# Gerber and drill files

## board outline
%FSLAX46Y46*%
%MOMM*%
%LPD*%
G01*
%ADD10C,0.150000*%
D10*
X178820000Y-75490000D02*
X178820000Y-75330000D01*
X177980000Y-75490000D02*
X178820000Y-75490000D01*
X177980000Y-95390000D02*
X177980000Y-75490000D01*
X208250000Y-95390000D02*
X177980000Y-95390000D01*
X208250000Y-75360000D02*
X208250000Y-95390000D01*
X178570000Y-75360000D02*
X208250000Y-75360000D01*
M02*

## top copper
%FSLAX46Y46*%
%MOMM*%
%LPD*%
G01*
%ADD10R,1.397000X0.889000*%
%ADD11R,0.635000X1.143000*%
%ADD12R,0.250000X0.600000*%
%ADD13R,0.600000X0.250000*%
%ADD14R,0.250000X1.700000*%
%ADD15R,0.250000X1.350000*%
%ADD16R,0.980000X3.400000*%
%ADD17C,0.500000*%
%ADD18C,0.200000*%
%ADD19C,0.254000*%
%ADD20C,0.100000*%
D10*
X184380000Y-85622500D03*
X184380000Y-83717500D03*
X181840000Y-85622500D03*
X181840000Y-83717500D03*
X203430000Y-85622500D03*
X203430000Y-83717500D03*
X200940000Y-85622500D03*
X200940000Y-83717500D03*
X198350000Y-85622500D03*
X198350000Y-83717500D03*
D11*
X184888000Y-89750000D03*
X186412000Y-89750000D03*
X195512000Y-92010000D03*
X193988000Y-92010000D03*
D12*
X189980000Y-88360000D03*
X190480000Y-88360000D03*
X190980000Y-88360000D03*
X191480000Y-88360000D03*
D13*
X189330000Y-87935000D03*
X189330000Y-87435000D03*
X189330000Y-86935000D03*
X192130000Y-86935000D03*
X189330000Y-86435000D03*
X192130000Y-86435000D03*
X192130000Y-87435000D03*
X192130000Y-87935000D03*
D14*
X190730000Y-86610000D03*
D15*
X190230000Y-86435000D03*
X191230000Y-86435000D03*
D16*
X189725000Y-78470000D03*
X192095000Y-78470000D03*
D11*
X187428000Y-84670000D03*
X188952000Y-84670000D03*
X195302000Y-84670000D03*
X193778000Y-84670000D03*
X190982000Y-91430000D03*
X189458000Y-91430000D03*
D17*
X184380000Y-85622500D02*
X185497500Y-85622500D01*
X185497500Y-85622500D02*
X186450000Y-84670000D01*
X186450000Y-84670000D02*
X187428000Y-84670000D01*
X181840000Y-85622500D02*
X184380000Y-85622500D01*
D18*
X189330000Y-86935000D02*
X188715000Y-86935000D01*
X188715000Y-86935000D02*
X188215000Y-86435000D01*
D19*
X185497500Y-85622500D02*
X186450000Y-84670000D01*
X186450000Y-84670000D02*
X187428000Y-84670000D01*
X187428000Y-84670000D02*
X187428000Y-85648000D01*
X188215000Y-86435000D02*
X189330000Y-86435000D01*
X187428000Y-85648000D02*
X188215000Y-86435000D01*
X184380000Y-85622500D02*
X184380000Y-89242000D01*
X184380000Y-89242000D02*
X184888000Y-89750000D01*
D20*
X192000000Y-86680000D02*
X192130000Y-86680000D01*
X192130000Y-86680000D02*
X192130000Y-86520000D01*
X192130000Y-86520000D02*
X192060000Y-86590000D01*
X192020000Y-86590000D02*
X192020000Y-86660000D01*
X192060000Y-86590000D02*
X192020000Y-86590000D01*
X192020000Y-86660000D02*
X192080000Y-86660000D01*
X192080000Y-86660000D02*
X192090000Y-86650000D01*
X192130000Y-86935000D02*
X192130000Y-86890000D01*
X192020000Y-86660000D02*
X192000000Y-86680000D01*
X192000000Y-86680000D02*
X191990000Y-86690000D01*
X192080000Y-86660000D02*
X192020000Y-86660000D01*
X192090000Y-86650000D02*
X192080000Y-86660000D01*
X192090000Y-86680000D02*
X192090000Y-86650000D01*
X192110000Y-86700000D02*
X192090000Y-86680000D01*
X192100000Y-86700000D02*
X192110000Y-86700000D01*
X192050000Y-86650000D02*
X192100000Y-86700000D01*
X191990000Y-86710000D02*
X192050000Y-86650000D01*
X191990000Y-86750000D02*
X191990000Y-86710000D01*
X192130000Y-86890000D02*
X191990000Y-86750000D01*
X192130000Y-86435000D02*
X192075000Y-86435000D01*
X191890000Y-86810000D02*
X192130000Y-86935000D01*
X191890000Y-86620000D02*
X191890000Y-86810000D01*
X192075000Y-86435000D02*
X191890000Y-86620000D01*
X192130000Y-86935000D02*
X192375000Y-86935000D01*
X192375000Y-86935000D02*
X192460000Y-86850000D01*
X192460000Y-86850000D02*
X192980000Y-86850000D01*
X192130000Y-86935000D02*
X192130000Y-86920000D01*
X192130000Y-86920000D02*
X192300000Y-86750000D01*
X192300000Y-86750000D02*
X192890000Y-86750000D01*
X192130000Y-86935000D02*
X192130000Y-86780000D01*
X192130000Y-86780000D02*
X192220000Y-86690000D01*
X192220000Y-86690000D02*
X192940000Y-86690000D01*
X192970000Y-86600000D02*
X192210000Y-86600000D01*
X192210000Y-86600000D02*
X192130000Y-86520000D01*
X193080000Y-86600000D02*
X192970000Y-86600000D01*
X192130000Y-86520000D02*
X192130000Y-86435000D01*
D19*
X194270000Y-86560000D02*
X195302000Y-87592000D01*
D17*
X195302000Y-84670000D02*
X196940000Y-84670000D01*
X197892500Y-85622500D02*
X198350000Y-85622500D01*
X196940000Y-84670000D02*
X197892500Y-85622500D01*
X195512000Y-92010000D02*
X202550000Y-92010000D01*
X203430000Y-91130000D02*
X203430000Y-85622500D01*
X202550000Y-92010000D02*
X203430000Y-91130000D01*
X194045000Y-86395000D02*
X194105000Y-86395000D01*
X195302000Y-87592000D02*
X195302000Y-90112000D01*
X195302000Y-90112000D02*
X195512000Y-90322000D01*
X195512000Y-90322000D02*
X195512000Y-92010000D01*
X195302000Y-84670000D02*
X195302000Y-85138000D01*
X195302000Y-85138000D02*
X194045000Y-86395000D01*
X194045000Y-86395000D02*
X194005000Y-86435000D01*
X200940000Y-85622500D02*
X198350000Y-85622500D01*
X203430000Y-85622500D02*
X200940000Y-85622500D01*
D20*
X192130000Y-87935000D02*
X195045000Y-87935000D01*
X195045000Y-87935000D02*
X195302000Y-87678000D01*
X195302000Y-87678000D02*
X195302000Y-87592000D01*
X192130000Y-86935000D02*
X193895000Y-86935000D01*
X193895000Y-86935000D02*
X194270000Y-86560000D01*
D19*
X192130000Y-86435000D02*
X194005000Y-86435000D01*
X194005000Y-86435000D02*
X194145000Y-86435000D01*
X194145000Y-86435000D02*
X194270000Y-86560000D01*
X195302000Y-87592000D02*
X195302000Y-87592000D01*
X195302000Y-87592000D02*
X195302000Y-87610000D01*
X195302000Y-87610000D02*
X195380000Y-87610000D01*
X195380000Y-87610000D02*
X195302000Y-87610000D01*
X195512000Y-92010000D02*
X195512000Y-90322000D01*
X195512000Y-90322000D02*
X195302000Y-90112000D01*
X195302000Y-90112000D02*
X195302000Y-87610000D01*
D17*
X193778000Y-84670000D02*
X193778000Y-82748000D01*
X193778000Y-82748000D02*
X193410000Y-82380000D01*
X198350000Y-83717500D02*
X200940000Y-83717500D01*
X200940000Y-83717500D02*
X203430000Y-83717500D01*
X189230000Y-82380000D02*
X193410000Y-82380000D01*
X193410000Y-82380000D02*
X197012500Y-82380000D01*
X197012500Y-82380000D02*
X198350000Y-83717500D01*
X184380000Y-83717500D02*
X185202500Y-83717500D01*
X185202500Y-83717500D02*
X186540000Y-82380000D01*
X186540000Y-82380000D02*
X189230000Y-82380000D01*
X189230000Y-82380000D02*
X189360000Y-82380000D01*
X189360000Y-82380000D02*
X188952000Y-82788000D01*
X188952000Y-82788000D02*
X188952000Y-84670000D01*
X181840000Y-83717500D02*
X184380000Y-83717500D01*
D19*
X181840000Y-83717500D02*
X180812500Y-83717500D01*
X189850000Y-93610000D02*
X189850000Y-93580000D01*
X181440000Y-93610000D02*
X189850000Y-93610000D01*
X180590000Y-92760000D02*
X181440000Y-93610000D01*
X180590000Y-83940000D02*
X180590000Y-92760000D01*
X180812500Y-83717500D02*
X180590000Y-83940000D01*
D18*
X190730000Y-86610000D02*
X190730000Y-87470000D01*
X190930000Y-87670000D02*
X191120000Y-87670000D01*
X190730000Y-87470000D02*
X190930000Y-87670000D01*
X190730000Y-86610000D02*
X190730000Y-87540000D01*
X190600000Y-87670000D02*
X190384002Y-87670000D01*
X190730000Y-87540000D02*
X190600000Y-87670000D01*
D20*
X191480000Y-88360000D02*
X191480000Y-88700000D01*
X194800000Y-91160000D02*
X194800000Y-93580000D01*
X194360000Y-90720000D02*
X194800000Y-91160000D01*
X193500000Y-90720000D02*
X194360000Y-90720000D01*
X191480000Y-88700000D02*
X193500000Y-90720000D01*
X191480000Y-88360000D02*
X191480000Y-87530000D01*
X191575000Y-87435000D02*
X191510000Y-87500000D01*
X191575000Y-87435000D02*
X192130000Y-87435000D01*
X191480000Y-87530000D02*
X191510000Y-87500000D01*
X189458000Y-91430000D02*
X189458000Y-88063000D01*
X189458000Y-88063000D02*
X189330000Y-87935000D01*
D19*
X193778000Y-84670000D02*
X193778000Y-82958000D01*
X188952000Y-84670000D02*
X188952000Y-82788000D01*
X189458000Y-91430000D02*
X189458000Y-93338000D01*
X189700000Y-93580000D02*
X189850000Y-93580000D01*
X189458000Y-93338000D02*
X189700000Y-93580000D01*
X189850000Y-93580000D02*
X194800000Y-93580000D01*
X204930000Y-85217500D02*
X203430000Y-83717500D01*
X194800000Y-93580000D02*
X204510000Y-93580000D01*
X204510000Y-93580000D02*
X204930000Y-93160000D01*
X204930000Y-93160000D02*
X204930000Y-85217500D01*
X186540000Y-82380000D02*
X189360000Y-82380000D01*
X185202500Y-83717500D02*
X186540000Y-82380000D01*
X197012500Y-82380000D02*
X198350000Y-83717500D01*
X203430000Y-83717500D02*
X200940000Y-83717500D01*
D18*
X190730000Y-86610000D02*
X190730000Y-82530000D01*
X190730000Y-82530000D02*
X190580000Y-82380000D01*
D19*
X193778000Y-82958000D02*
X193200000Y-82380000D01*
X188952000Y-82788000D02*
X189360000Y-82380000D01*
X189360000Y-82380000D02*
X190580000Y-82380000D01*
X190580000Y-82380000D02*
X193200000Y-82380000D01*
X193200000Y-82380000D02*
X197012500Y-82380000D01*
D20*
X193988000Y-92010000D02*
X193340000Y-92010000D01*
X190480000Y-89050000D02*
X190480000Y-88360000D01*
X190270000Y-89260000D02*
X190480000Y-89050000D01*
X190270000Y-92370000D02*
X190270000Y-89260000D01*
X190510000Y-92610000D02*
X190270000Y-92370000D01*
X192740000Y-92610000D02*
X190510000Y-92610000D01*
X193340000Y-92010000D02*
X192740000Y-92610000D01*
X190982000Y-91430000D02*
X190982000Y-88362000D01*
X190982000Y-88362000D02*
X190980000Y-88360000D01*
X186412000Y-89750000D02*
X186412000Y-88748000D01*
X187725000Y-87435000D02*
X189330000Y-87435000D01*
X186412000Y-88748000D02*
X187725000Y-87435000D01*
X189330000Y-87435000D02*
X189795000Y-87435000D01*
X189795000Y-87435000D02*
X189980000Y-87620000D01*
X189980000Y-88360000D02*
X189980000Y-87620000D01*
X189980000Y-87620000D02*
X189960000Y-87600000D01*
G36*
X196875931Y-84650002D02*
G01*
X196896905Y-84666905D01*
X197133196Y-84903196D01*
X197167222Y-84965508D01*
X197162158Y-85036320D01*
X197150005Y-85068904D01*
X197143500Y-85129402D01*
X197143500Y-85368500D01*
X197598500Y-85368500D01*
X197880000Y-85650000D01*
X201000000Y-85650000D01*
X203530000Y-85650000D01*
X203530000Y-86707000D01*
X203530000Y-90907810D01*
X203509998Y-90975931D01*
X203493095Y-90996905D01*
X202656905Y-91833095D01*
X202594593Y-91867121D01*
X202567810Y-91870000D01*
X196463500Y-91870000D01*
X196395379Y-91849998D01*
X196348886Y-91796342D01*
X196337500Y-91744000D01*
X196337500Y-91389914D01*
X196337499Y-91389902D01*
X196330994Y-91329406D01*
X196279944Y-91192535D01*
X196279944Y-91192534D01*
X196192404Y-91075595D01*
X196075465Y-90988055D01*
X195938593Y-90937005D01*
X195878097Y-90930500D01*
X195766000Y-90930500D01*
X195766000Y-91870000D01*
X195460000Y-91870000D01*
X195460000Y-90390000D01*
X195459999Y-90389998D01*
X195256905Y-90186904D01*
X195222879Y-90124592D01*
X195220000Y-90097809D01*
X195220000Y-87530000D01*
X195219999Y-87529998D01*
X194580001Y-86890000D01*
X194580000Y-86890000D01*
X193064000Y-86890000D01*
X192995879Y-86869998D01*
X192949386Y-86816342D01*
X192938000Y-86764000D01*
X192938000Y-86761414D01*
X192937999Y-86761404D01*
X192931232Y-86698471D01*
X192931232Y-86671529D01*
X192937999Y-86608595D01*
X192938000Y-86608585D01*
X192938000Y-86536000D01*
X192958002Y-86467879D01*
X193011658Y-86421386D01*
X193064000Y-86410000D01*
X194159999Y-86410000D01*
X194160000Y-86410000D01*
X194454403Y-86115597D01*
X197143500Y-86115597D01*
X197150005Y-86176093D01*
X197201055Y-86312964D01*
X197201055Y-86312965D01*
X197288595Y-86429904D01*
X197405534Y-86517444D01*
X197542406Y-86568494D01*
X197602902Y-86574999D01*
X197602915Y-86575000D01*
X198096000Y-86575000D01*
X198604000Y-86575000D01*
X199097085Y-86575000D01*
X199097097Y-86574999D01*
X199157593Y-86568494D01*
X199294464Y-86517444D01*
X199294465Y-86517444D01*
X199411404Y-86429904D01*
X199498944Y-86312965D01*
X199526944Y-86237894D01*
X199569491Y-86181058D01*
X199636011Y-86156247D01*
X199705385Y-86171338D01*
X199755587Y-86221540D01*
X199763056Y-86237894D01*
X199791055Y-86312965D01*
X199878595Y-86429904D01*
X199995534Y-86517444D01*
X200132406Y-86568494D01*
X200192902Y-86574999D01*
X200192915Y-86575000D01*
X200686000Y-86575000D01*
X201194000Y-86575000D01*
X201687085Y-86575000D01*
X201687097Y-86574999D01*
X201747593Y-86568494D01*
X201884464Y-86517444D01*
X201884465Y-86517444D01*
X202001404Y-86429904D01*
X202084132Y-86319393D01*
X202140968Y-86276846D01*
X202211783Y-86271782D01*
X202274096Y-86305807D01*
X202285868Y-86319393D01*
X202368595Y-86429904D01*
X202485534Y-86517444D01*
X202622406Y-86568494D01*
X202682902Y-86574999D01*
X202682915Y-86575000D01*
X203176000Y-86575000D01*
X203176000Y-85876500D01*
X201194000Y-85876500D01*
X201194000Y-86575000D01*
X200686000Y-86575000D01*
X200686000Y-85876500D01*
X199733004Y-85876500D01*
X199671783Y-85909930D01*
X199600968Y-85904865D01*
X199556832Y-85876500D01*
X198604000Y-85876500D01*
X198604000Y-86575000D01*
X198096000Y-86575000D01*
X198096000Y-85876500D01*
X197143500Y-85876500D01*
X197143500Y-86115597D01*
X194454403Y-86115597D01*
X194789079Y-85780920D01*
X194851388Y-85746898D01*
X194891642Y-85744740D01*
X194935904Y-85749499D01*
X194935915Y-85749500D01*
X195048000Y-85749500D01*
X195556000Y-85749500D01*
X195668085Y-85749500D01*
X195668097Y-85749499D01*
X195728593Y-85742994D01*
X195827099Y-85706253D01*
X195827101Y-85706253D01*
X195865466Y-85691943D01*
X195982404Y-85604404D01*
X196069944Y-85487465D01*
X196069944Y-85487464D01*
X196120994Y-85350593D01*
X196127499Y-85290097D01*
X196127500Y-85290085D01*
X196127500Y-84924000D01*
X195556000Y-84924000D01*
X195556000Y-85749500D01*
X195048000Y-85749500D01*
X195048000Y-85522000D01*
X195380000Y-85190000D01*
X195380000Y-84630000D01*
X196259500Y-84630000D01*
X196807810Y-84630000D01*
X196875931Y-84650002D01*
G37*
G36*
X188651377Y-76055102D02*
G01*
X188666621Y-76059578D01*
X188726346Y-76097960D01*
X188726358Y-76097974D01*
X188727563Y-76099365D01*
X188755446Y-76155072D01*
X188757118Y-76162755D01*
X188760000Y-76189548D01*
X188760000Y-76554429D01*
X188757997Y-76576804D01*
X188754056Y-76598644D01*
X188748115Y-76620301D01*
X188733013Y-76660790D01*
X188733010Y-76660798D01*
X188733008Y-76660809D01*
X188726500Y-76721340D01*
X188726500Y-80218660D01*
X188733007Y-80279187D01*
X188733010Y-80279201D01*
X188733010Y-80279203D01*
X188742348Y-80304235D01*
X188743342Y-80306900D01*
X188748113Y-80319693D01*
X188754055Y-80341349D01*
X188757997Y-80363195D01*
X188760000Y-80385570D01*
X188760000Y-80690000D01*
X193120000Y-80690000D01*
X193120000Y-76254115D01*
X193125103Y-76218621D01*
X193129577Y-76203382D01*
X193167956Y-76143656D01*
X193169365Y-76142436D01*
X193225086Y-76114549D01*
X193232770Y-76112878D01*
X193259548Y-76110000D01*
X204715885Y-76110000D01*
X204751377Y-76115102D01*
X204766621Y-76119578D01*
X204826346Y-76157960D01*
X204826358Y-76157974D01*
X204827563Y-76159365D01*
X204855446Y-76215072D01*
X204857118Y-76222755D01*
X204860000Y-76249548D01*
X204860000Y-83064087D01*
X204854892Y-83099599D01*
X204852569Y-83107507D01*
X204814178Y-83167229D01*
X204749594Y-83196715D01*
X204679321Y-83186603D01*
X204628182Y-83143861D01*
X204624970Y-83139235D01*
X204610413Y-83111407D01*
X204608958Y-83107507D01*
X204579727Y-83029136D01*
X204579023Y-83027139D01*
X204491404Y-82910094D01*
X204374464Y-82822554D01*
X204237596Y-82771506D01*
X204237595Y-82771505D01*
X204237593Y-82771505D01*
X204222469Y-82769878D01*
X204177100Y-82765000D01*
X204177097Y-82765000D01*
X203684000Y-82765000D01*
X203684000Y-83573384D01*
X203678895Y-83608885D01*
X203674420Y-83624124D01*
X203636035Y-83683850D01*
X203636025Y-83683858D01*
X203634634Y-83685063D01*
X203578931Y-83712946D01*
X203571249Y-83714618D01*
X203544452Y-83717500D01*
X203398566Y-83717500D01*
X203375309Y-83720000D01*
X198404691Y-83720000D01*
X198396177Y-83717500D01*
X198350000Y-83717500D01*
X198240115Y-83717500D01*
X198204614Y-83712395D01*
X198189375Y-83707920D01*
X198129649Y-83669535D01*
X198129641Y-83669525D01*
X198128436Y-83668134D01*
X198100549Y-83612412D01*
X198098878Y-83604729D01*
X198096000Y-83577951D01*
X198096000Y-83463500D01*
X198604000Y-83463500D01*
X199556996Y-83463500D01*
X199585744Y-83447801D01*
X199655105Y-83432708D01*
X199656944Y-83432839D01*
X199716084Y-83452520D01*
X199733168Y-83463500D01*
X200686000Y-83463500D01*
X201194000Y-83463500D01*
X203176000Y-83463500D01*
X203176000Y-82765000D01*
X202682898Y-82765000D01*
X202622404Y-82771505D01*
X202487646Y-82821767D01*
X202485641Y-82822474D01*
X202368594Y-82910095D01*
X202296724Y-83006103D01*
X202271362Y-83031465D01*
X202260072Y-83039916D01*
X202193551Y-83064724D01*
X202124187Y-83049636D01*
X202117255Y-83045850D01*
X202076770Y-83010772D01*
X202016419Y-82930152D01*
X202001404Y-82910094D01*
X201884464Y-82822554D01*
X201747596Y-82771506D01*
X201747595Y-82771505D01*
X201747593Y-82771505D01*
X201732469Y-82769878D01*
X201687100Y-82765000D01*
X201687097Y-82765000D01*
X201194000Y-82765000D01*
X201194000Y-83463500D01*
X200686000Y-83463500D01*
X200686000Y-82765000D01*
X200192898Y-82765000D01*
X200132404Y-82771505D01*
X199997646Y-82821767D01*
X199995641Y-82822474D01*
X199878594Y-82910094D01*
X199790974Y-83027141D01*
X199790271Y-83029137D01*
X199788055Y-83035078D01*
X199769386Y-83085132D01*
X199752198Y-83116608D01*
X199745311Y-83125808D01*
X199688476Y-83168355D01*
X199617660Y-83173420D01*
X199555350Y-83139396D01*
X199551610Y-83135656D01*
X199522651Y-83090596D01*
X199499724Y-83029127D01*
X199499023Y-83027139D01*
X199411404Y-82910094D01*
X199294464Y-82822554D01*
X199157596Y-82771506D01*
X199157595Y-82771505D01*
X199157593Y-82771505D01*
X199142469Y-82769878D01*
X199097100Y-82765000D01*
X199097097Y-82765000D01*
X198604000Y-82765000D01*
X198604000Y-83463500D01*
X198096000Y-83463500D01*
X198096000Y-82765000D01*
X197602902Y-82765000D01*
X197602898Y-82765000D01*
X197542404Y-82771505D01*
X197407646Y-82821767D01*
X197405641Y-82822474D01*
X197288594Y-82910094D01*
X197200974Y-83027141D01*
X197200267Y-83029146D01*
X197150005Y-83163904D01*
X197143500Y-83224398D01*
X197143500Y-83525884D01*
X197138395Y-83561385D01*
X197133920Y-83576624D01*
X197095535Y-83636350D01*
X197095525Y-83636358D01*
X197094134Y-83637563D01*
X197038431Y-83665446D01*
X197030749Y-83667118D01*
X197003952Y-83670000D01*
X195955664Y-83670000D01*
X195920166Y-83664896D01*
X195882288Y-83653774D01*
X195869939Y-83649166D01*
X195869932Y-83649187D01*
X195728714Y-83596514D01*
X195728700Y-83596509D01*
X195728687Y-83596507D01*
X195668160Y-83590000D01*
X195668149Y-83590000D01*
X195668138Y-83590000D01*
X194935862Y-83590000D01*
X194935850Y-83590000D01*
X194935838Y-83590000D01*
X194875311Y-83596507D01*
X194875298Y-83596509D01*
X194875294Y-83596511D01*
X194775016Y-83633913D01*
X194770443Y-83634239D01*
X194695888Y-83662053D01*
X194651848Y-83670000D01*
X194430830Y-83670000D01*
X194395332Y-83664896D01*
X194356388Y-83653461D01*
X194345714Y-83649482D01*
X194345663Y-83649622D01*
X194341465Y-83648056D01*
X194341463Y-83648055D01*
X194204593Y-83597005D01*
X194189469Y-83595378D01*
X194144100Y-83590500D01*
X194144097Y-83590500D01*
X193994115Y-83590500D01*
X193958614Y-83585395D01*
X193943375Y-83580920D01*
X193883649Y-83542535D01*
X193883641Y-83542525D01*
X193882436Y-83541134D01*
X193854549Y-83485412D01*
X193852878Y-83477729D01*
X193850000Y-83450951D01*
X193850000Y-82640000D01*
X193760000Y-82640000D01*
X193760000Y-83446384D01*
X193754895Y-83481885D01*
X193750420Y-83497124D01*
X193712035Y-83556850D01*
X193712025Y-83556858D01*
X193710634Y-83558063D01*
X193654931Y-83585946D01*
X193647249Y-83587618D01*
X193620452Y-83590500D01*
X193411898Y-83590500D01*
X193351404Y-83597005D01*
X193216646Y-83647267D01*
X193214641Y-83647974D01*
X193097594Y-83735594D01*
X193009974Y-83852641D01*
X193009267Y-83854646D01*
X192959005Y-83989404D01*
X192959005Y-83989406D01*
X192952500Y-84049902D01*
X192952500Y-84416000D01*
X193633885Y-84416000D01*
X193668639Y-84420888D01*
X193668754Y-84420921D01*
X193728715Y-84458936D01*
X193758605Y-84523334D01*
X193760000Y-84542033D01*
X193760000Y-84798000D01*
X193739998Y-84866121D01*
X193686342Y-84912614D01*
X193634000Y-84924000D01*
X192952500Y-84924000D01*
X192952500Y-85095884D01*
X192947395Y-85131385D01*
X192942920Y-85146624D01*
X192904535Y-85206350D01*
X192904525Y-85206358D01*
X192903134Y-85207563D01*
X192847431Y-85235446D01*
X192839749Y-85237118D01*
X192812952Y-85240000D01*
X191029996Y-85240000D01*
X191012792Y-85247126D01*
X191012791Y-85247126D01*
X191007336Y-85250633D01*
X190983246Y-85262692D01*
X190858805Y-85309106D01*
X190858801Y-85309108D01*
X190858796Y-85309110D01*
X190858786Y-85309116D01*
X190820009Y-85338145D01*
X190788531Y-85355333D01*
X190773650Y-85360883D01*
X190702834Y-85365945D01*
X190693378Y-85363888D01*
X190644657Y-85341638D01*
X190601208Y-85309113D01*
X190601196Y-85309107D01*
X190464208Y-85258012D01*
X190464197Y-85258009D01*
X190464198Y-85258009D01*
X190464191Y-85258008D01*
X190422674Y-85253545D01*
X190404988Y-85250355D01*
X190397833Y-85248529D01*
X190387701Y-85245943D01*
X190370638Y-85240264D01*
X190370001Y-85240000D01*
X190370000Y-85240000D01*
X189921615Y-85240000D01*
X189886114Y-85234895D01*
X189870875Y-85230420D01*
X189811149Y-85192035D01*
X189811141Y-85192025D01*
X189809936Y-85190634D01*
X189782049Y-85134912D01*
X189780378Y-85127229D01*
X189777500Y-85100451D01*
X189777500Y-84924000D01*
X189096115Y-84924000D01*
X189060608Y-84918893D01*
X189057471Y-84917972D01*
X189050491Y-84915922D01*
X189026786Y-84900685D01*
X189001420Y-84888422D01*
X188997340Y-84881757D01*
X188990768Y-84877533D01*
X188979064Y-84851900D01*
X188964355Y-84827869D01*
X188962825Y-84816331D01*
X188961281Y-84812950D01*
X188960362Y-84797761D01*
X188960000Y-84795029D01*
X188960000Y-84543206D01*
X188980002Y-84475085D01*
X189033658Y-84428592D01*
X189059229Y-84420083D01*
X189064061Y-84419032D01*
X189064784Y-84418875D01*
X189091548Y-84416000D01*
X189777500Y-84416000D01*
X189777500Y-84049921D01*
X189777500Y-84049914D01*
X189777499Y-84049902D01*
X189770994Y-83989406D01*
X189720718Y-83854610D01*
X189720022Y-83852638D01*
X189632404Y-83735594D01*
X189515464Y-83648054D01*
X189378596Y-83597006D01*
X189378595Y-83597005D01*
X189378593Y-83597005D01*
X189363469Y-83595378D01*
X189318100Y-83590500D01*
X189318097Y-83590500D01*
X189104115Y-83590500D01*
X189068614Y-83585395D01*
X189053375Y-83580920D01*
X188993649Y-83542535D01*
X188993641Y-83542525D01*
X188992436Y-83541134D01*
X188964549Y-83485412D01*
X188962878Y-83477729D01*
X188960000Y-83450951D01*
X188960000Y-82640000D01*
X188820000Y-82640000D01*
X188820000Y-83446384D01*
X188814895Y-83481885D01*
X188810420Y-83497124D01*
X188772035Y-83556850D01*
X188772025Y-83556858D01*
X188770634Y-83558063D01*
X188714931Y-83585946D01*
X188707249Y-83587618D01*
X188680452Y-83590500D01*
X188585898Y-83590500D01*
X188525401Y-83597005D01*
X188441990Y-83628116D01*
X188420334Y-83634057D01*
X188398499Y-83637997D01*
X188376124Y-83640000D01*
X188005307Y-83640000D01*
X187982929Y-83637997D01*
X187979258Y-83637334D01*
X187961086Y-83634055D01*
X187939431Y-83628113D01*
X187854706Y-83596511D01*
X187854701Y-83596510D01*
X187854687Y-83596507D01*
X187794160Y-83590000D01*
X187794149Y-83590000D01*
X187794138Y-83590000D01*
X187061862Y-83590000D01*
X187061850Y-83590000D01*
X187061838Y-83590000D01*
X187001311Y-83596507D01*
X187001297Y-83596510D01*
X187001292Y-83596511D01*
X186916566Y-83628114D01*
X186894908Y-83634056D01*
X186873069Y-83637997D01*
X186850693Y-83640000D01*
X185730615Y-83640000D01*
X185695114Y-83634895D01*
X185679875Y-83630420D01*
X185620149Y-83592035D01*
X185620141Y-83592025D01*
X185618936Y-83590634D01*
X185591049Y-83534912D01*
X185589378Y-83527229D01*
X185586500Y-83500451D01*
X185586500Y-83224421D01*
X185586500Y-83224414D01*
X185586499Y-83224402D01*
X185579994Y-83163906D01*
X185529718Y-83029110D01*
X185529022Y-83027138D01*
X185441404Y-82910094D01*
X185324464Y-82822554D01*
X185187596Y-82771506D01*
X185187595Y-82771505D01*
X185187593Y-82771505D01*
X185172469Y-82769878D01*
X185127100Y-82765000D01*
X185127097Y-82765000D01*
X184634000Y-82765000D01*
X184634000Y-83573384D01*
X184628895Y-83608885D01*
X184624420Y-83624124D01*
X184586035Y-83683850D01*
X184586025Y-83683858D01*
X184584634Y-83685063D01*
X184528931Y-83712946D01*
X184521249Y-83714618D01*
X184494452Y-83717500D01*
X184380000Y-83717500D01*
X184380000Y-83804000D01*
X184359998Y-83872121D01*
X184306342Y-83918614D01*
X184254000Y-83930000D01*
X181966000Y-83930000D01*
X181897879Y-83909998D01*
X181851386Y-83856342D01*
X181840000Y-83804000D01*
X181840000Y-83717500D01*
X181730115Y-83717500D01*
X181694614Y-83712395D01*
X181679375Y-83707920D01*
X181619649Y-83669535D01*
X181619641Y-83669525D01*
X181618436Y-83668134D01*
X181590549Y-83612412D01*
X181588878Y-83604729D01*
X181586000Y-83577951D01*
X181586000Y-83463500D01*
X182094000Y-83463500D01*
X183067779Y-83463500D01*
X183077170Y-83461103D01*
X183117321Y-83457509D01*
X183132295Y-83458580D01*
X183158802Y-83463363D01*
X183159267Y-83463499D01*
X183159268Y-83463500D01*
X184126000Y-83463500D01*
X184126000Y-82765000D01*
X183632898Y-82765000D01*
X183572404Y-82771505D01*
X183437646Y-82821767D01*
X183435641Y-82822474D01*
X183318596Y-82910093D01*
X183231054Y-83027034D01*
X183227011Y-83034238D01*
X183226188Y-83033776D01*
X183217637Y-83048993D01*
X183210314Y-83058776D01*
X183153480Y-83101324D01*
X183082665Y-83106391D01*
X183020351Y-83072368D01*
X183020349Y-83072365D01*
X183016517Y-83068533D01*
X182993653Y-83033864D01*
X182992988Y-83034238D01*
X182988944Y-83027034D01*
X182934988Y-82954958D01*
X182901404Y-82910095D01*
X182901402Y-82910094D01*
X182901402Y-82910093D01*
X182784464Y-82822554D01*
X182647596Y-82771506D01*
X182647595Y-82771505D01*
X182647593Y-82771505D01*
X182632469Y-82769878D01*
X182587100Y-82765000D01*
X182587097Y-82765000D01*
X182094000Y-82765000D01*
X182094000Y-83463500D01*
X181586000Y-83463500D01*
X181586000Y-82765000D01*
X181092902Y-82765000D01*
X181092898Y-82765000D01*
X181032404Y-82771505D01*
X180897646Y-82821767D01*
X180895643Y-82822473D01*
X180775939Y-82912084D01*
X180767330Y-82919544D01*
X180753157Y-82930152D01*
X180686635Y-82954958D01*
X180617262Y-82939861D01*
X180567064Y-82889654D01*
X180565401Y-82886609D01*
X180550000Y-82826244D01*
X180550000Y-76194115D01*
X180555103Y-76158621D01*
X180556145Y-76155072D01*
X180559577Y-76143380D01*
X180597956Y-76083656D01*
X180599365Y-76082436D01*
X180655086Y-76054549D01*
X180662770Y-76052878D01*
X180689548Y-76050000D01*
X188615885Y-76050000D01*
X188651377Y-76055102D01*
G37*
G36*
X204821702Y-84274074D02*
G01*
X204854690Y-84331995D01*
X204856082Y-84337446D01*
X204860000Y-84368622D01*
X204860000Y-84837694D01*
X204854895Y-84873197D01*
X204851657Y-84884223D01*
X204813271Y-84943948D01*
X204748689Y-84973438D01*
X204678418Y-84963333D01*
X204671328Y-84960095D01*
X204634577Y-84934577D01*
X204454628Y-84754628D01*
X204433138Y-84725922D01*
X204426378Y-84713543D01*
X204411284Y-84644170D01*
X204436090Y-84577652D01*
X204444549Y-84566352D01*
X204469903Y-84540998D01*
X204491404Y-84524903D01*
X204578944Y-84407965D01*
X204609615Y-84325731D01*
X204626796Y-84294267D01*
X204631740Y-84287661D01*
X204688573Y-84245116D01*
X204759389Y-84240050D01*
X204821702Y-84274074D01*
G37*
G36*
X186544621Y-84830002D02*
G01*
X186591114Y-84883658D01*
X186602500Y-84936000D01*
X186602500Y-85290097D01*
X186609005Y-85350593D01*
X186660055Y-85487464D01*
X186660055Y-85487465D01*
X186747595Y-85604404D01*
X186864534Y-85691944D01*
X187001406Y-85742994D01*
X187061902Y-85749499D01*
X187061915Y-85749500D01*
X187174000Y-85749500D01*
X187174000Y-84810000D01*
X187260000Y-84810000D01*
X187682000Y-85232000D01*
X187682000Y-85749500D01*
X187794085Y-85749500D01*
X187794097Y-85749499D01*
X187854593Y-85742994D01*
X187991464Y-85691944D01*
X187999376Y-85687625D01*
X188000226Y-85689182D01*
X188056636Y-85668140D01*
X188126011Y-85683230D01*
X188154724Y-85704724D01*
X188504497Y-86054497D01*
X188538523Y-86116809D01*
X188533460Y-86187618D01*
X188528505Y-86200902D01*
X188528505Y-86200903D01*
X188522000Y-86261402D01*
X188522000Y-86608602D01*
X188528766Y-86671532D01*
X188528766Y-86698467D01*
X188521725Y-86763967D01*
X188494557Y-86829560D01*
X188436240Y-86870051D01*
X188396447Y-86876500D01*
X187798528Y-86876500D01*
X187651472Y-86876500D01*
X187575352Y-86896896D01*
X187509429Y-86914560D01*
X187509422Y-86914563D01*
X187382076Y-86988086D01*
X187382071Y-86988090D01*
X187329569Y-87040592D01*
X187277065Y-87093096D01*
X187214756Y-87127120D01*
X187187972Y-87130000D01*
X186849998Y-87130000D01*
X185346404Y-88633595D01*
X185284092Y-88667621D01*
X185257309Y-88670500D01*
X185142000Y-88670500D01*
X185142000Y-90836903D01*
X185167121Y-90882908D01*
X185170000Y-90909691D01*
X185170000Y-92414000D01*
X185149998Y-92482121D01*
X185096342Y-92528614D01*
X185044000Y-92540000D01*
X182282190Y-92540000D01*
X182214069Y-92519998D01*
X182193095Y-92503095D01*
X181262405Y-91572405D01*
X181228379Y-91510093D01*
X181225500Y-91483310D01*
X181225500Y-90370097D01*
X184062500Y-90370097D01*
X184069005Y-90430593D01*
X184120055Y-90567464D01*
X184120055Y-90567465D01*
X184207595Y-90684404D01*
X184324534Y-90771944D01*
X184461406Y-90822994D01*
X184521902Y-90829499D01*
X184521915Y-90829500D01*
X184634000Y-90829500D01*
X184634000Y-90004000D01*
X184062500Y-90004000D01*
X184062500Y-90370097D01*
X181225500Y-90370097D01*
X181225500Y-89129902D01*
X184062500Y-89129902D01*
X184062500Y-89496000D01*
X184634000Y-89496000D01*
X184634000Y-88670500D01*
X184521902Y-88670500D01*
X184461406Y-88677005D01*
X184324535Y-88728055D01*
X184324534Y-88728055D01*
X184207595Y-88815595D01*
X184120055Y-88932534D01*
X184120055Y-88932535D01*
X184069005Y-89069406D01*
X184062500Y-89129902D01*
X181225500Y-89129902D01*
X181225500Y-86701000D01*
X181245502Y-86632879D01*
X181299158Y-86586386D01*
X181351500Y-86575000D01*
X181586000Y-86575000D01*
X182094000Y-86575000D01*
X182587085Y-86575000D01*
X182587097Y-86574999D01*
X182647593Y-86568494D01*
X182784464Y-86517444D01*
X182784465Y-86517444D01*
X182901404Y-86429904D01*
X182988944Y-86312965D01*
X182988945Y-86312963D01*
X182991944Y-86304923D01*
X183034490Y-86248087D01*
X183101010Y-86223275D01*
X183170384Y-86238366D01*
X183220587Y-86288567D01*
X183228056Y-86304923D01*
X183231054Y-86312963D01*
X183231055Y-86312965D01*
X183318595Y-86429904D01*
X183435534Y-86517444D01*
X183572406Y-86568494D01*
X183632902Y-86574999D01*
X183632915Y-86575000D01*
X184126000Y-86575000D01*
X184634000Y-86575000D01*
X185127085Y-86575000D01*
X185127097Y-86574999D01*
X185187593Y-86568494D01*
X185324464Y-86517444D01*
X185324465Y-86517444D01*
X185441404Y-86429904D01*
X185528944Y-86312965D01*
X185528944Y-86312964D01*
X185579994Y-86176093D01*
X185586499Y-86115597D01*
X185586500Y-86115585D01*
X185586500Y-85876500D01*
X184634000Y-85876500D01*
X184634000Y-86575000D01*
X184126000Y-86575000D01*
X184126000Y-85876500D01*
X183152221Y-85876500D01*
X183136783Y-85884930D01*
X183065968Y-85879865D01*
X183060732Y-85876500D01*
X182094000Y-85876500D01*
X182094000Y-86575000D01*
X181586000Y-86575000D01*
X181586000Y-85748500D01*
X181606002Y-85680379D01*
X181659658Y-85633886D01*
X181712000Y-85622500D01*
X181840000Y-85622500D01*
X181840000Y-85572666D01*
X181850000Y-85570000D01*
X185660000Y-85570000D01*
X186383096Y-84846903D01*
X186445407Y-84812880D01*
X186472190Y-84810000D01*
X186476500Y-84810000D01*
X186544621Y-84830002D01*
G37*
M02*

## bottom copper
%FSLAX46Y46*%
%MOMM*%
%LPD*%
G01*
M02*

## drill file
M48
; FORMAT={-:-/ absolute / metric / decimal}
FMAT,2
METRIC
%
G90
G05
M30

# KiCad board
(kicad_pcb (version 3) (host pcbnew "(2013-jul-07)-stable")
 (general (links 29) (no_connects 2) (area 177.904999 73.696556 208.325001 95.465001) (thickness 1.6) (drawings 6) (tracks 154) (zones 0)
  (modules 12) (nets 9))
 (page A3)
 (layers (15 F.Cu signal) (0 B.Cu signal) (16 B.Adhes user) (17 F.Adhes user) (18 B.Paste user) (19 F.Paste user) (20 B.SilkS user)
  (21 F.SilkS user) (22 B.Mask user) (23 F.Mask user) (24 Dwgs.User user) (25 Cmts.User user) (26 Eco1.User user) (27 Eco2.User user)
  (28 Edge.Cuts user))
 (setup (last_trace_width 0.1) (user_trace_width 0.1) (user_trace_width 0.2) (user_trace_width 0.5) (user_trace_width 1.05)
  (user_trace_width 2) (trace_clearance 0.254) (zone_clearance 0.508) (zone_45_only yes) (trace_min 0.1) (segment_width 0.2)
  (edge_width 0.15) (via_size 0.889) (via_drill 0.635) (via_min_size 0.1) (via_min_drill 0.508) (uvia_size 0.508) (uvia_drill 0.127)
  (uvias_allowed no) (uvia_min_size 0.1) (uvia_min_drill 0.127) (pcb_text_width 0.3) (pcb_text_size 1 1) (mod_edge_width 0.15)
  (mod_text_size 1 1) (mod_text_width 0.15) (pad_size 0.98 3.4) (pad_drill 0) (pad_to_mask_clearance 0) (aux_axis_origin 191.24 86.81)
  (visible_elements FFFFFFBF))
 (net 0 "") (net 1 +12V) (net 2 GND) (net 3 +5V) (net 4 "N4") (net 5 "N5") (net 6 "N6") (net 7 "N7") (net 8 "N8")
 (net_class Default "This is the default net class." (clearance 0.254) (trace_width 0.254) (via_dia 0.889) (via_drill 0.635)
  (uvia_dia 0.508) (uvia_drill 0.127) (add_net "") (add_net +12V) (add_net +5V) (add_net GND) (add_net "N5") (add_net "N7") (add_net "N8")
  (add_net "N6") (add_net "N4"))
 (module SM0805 (layer F.Cu) (at 184.38 84.67 90)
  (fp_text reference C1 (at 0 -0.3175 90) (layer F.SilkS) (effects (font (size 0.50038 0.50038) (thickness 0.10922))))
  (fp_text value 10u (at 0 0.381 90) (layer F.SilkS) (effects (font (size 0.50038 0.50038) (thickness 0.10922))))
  (pad 1 smd rect (at -0.9525 0 90) (size 0.889 1.397) (layers F.Cu F.Paste F.Mask) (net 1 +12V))
  (pad 2 smd rect (at 0.9525 0 90) (size 0.889 1.397) (layers F.Cu F.Paste F.Mask) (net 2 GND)))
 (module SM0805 (layer F.Cu) (at 181.84 84.67 90)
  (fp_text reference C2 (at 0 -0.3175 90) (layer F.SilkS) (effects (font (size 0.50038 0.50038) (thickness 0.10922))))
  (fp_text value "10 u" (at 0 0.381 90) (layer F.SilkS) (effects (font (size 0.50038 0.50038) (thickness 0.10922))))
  (pad 1 smd rect (at -0.9525 0 90) (size 0.889 1.397) (layers F.Cu F.Paste F.Mask) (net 1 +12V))
  (pad 2 smd rect (at 0.9525 0 90) (size 0.889 1.397) (layers F.Cu F.Paste F.Mask) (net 2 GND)))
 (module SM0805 (layer F.Cu) (at 203.43 84.67 90)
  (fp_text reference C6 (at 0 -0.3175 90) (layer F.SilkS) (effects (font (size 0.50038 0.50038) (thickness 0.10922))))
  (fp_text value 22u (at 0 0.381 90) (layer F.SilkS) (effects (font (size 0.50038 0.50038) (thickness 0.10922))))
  (pad 1 smd rect (at -0.9525 0 90) (size 0.889 1.397) (layers F.Cu F.Paste F.Mask) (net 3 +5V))
  (pad 2 smd rect (at 0.9525 0 90) (size 0.889 1.397) (layers F.Cu F.Paste F.Mask) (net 2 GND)))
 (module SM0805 (layer F.Cu) (at 200.94 84.67 90)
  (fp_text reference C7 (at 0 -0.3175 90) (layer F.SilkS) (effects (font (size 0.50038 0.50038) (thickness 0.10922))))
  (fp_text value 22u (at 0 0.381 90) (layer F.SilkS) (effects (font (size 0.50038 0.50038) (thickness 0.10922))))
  (pad 1 smd rect (at -0.9525 0 90) (size 0.889 1.397) (layers F.Cu F.Paste F.Mask) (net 3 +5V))
  (pad 2 smd rect (at 0.9525 0 90) (size 0.889 1.397) (layers F.Cu F.Paste F.Mask) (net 2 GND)))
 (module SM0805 (layer F.Cu) (at 198.35 84.67 90)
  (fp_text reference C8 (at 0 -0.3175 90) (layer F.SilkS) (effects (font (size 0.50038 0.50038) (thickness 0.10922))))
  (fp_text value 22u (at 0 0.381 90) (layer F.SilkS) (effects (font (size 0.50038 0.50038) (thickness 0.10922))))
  (pad 1 smd rect (at -0.9525 0 90) (size 0.889 1.397) (layers F.Cu F.Paste F.Mask) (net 3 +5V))
  (pad 2 smd rect (at 0.9525 0 90) (size 0.889 1.397) (layers F.Cu F.Paste F.Mask) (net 2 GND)))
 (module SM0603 (layer F.Cu) (at 185.65 89.75)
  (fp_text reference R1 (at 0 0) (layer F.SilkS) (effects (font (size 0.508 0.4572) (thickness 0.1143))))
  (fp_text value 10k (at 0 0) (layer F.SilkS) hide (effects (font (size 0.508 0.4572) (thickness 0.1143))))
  (pad 1 smd rect (at -0.762 0) (size 0.635 1.143) (layers F.Cu F.Paste F.Mask) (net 1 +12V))
  (pad 2 smd rect (at 0.762 0) (size 0.635 1.143) (layers F.Cu F.Paste F.Mask) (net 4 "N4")))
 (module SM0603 (layer F.Cu) (at 194.75 92.01 180)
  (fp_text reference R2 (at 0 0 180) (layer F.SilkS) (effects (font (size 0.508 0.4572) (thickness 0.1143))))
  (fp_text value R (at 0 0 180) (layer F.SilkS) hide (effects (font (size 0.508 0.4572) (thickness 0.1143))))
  (pad 1 smd rect (at -0.762 0 180) (size 0.635 1.143) (layers F.Cu F.Paste F.Mask) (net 3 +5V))
  (pad 2 smd rect (at 0.762 0 180) (size 0.635 1.143) (layers F.Cu F.Paste F.Mask) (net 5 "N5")))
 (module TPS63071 (layer F.Cu) (at 190.73 87.21 90)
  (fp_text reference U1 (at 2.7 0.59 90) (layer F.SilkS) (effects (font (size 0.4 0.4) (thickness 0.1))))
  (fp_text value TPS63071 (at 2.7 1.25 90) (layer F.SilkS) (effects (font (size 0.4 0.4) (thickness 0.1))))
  (pad 1 smd rect (at -1.15 -0.75 90) (size 0.6 0.25) (layers F.Cu F.Paste F.Mask) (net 4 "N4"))
  (pad 2 smd rect (at -1.15 -0.25 90) (size 0.6 0.25) (layers F.Cu F.Paste F.Mask) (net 5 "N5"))
  (pad 3 smd rect (at -1.15 0.25 90) (size 0.6 0.25) (layers F.Cu F.Paste F.Mask) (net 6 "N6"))
  (pad 4 smd rect (at -1.15 0.75 90) (size 0.6 0.25) (layers F.Cu F.Paste F.Mask) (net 2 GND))
  (pad 15 smd rect (at -0.725 -1.4 90) (size 0.25 0.6) (layers F.Cu F.Paste F.Mask) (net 2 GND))
  (pad 14 smd rect (at -0.225 -1.4 90) (size 0.25 0.6) (layers F.Cu F.Paste F.Mask) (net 4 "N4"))
  (pad 13 smd rect (at 0.275 -1.4 90) (size 0.25 0.6) (layers F.Cu F.Paste F.Mask) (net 1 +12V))
  (pad 7 smd rect (at 0.275 1.4 90) (size 0.25 0.6) (layers F.Cu F.Paste F.Mask) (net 3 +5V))
  (pad 12 smd rect (at 0.775 -1.4 90) (size 0.25 0.6) (layers F.Cu F.Paste F.Mask) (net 1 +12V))
  (pad 8 smd rect (at 0.775 1.4 90) (size 0.25 0.6) (layers F.Cu F.Paste F.Mask) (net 3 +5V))
  (pad 6 smd rect (at -0.225 1.4 90) (size 0.25 0.6) (layers F.Cu F.Paste F.Mask) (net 2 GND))
  (pad 5 smd rect (at -0.725 1.4 90) (size 0.25 0.6) (layers F.Cu F.Paste F.Mask) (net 3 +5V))
  (pad 10 smd rect (at 0.6 0 90) (size 1.7 0.25) (layers F.Cu F.Paste F.Mask) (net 2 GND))
  (pad 11 smd rect (at 0.775 -0.5 90) (size 1.35 0.25) (layers F.Cu F.Paste F.Mask) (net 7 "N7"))
  (pad 9 smd rect (at 0.775 0.5 90) (size 1.35 0.25) (layers F.Cu F.Paste F.Mask) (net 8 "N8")))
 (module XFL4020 (layer F.Cu) (at 190.91 78.47)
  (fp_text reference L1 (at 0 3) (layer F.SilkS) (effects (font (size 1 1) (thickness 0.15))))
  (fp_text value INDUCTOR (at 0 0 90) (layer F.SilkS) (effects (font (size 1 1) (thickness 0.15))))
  (pad 1 smd rect (at -1.185 0) (size 0.98 3.4) (layers F.Cu F.Paste F.Mask) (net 7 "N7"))
  (pad 2 smd rect (at 1.185 0) (size 0.98 3.4) (layers F.Cu F.Paste F.Mask) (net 8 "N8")))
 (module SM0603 (layer F.Cu) (at 188.19 84.67)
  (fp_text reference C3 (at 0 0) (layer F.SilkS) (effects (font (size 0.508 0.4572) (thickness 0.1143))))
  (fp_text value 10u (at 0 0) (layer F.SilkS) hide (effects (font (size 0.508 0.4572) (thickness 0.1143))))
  (pad 1 smd rect (at -0.762 0) (size 0.635 1.143) (layers F.Cu F.Paste F.Mask) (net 1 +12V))
  (pad 2 smd rect (at 0.762 0) (size 0.635 1.143) (layers F.Cu F.Paste F.Mask) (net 2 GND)))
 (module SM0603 (layer F.Cu) (at 194.54 84.67 180)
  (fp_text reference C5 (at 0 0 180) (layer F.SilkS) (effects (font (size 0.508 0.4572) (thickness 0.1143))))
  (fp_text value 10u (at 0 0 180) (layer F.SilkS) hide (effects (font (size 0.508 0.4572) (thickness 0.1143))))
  (pad 1 smd rect (at -0.762 0 180) (size 0.635 1.143) (layers F.Cu F.Paste F.Mask) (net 3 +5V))
  (pad 2 smd rect (at 0.762 0 180) (size 0.635 1.143) (layers F.Cu F.Paste F.Mask) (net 2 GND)))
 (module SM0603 (layer F.Cu) (at 190.22 91.43 180)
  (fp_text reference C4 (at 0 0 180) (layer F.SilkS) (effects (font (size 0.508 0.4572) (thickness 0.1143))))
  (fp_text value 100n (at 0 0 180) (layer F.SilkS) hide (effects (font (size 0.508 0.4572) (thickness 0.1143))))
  (pad 1 smd rect (at -0.762 0 180) (size 0.635 1.143) (layers F.Cu F.Paste F.Mask) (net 6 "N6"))
  (pad 2 smd rect (at 0.762 0 180) (size 0.635 1.143) (layers F.Cu F.Paste F.Mask) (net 2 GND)))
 (gr_line (start 178.82 75.49) (end 178.82 75.33) (angle 90) (layer Edge.Cuts) (width 0.15))
 (gr_line (start 177.98 75.49) (end 178.82 75.49) (angle 90) (layer Edge.Cuts) (width 0.15))
 (gr_line (start 177.98 95.39) (end 177.98 75.49) (angle 90) (layer Edge.Cuts) (width 0.15))
 (gr_line (start 208.25 95.39) (end 177.98 95.39) (angle 90) (layer Edge.Cuts) (width 0.15))
 (gr_line (start 208.25 75.36) (end 208.25 95.39) (angle 90) (layer Edge.Cuts) (width 0.15))
 (gr_line (start 178.57 75.36) (end 208.25 75.36) (angle 90) (layer Edge.Cuts) (width 0.15))
 (segment (start 184.38 85.6225) (end 185.4975 85.6225) (width 0.5) (layer F.Cu) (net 1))
 (segment (start 185.4975 85.6225) (end 186.45 84.67) (width 0.5) (layer F.Cu) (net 1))
 (segment (start 186.45 84.67) (end 187.428 84.67) (width 0.5) (layer F.Cu) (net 1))
 (segment (start 181.84 85.6225) (end 184.38 85.6225) (width 0.5) (layer F.Cu) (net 1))
 (segment (start 189.33 86.935) (end 188.715 86.935) (width 0.2) (layer F.Cu) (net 1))
 (segment (start 188.715 86.935) (end 188.215 86.435) (width 0.2) (layer F.Cu) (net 1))
 (segment (start 185.4975 85.6225) (end 186.45 84.67) (width 0.254) (layer F.Cu) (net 1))
 (segment (start 186.45 84.67) (end 187.428 84.67) (width 0.254) (layer F.Cu) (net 1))
 (segment (start 187.428 84.67) (end 187.428 85.648) (width 0.254) (layer F.Cu) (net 1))
 (segment (start 188.215 86.435) (end 189.33 86.435) (width 0.254) (layer F.Cu) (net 1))
 (segment (start 187.428 85.648) (end 188.215 86.435) (width 0.254) (layer F.Cu) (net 1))
 (segment (start 184.38 85.6225) (end 184.38 89.242) (width 0.254) (layer F.Cu) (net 1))
 (segment (start 184.38 89.242) (end 184.888 89.75) (width 0.254) (layer F.Cu) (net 1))
 (segment (start 192 86.68) (end 192.13 86.68) (width 0.1) (layer F.Cu) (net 3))
 (segment (start 192.13 86.68) (end 192.13 86.52) (width 0.1) (layer F.Cu) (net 3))
 (segment (start 192.13 86.52) (end 192.06 86.59) (width 0.1) (layer F.Cu) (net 3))
 (segment (start 192.02 86.59) (end 192.02 86.66) (width 0.1) (layer F.Cu) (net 3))
 (segment (start 192.06 86.59) (end 192.02 86.59) (width 0.1) (layer F.Cu) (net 3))
 (segment (start 192.02 86.66) (end 192.08 86.66) (width 0.1) (layer F.Cu) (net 3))
 (segment (start 192.08 86.66) (end 192.09 86.65) (width 0.1) (layer F.Cu) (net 3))
 (segment (start 192.13 86.935) (end 192.13 86.89) (width 0.1) (layer F.Cu) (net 3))
 (segment (start 192.02 86.66) (end 192 86.68) (width 0.1) (layer F.Cu) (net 3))
 (segment (start 192 86.68) (end 191.99 86.69) (width 0.1) (layer F.Cu) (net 3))
 (segment (start 192.08 86.66) (end 192.02 86.66) (width 0.1) (layer F.Cu) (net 3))
 (segment (start 192.09 86.65) (end 192.08 86.66) (width 0.1) (layer F.Cu) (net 3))
 (segment (start 192.09 86.68) (end 192.09 86.65) (width 0.1) (layer F.Cu) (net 3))
 (segment (start 192.11 86.7) (end 192.09 86.68) (width 0.1) (layer F.Cu) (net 3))
 (segment (start 192.1 86.7) (end 192.11 86.7) (width 0.1) (layer F.Cu) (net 3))
 (segment (start 192.05 86.65) (end 192.1 86.7) (width 0.1) (layer F.Cu) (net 3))
 (segment (start 191.99 86.71) (end 192.05 86.65) (width 0.1) (layer F.Cu) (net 3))
 (segment (start 191.99 86.75) (end 191.99 86.71) (width 0.1) (layer F.Cu) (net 3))
 (segment (start 192.13 86.89) (end 191.99 86.75) (width 0.1) (layer F.Cu) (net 3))
 (segment (start 192.13 86.435) (end 192.075 86.435) (width 0.1) (layer F.Cu) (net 3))
 (segment (start 191.89 86.81) (end 192.13 86.935) (width 0.1) (layer F.Cu) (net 3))
 (segment (start 191.89 86.62) (end 191.89 86.81) (width 0.1) (layer F.Cu) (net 3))
 (segment (start 192.075 86.435) (end 191.89 86.62) (width 0.1) (layer F.Cu) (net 3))
 (segment (start 192.13 86.935) (end 192.375 86.935) (width 0.1) (layer F.Cu) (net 3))
 (segment (start 192.375 86.935) (end 192.46 86.85) (width 0.1) (layer F.Cu) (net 3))
 (segment (start 192.46 86.85) (end 192.98 86.85) (width 0.1) (layer F.Cu) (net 3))
 (segment (start 192.13 86.935) (end 192.13 86.92) (width 0.1) (layer F.Cu) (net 3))
 (segment (start 192.13 86.92) (end 192.3 86.75) (width 0.1) (layer F.Cu) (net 3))
 (segment (start 192.3 86.75) (end 192.89 86.75) (width 0.1) (layer F.Cu) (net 3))
 (segment (start 192.13 86.935) (end 192.13 86.78) (width 0.1) (layer F.Cu) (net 3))
 (segment (start 192.13 86.78) (end 192.22 86.69) (width 0.1) (layer F.Cu) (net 3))
 (segment (start 192.22 86.69) (end 192.94 86.69) (width 0.1) (layer F.Cu) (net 3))
 (segment (start 192.97 86.6) (end 192.21 86.6) (width 0.1) (layer F.Cu) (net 3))
 (segment (start 192.21 86.6) (end 192.13 86.52) (width 0.1) (layer F.Cu) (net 3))
 (segment (start 193.08 86.6) (end 192.97 86.6) (width 0.1) (layer F.Cu) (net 3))
 (segment (start 192.13 86.52) (end 192.13 86.435) (width 0.1) (layer F.Cu) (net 3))
 (segment (start 194.27 86.56) (end 195.302 87.592) (width 0.254) (layer F.Cu) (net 3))
 (segment (start 195.302 84.67) (end 196.94 84.67) (width 0.5) (layer F.Cu) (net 3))
 (segment (start 197.8925 85.6225) (end 198.35 85.6225) (width 0.5) (layer F.Cu) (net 3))
 (segment (start 196.94 84.67) (end 197.8925 85.6225) (width 0.5) (layer F.Cu) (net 3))
 (segment (start 195.512 92.01) (end 202.55 92.01) (width 0.5) (layer F.Cu) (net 3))
 (segment (start 203.43 91.13) (end 203.43 85.6225) (width 0.5) (layer F.Cu) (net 3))
 (segment (start 202.55 92.01) (end 203.43 91.13) (width 0.5) (layer F.Cu) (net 3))
 (segment (start 194.045 86.395) (end 194.105 86.395) (width 0.5) (layer F.Cu) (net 3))
 (segment (start 195.302 87.592) (end 195.302 90.112) (width 0.5) (layer F.Cu) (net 3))
 (segment (start 195.302 90.112) (end 195.512 90.322) (width 0.5) (layer F.Cu) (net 3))
 (segment (start 195.512 90.322) (end 195.512 92.01) (width 0.5) (layer F.Cu) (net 3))
 (segment (start 195.302 84.67) (end 195.302 85.138) (width 0.5) (layer F.Cu) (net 3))
 (segment (start 195.302 85.138) (end 194.045 86.395) (width 0.5) (layer F.Cu) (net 3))
 (segment (start 194.045 86.395) (end 194.005 86.435) (width 0.5) (layer F.Cu) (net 3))
 (segment (start 200.94 85.6225) (end 198.35 85.6225) (width 0.5) (layer F.Cu) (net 3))
 (segment (start 203.43 85.6225) (end 200.94 85.6225) (width 0.5) (layer F.Cu) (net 3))
 (segment (start 192.13 87.935) (end 195.045 87.935) (width 0.1) (layer F.Cu) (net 3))
 (segment (start 195.045 87.935) (end 195.302 87.678) (width 0.1) (layer F.Cu) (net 3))
 (segment (start 195.302 87.678) (end 195.302 87.592) (width 0.1) (layer F.Cu) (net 3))
 (segment (start 192.13 86.935) (end 193.895 86.935) (width 0.1) (layer F.Cu) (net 3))
 (segment (start 193.895 86.935) (end 194.27 86.56) (width 0.1) (layer F.Cu) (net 3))
 (segment (start 192.13 86.435) (end 194.005 86.435) (width 0.254) (layer F.Cu) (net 3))
 (segment (start 194.005 86.435) (end 194.145 86.435) (width 0.254) (layer F.Cu) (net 3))
 (segment (start 194.145 86.435) (end 194.27 86.56) (width 0.254) (layer F.Cu) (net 3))
 (segment (start 195.302 87.592) (end 195.302 87.592) (width 0.254) (layer F.Cu) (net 3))
 (segment (start 195.302 87.592) (end 195.302 87.61) (width 0.254) (layer F.Cu) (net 3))
 (segment (start 195.302 87.61) (end 195.38 87.61) (width 0.254) (layer F.Cu) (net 3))
 (segment (start 195.38 87.61) (end 195.302 87.61) (width 0.254) (layer F.Cu) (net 3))
 (segment (start 195.512 92.01) (end 195.512 90.322) (width 0.254) (layer F.Cu) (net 3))
 (segment (start 195.512 90.322) (end 195.302 90.112) (width 0.254) (layer F.Cu) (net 3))
 (segment (start 195.302 90.112) (end 195.302 87.61) (width 0.254) (layer F.Cu) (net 3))
 (segment (start 193.778 84.67) (end 193.778 82.748) (width 0.5) (layer F.Cu) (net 2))
 (segment (start 193.778 82.748) (end 193.41 82.38) (width 0.5) (layer F.Cu) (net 2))
 (segment (start 198.35 83.7175) (end 200.94 83.7175) (width 0.5) (layer F.Cu) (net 2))
 (segment (start 200.94 83.7175) (end 203.43 83.7175) (width 0.5) (layer F.Cu) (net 2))
 (segment (start 189.23 82.38) (end 193.41 82.38) (width 0.5) (layer F.Cu) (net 2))
 (segment (start 193.41 82.38) (end 197.0125 82.38) (width 0.5) (layer F.Cu) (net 2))
 (segment (start 197.0125 82.38) (end 198.35 83.7175) (width 0.5) (layer F.Cu) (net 2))
 (segment (start 184.38 83.7175) (end 185.2025 83.7175) (width 0.5) (layer F.Cu) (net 2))
 (segment (start 185.2025 83.7175) (end 186.54 82.38) (width 0.5) (layer F.Cu) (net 2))
 (segment (start 186.54 82.38) (end 189.23 82.38) (width 0.5) (layer F.Cu) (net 2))
 (segment (start 189.23 82.38) (end 189.36 82.38) (width 0.5) (layer F.Cu) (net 2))
 (segment (start 189.36 82.38) (end 188.952 82.788) (width 0.5) (layer F.Cu) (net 2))
 (segment (start 188.952 82.788) (end 188.952 84.67) (width 0.5) (layer F.Cu) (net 2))
 (segment (start 181.84 83.7175) (end 184.38 83.7175) (width 0.5) (layer F.Cu) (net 2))
 (segment (start 181.84 83.7175) (end 180.8125 83.7175) (width 0.254) (layer F.Cu) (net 2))
 (segment (start 189.85 93.61) (end 189.85 93.58) (width 0.254) (layer F.Cu) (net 2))
 (segment (start 181.44 93.61) (end 189.85 93.61) (width 0.254) (layer F.Cu) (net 2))
 (segment (start 180.59 92.76) (end 181.44 93.61) (width 0.254) (layer F.Cu) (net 2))
 (segment (start 180.59 83.94) (end 180.59 92.76) (width 0.254) (layer F.Cu) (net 2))
 (segment (start 180.8125 83.7175) (end 180.59 83.94) (width 0.254) (layer F.Cu) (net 2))
 (segment (start 190.73 86.61) (end 190.73 87.47) (width 0.2) (layer F.Cu) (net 2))
 (segment (start 190.93 87.67) (end 191.12 87.67) (width 0.2) (layer F.Cu) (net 2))
 (segment (start 190.73 87.47) (end 190.93 87.67) (width 0.2) (layer F.Cu) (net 2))
 (segment (start 190.73 86.61) (end 190.73 87.54) (width 0.2) (layer F.Cu) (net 2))
 (segment (start 190.6 87.67) (end 190.384002 87.67) (width 0.2) (layer F.Cu) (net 2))
 (segment (start 190.73 87.54) (end 190.6 87.67) (width 0.2) (layer F.Cu) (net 2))
 (segment (start 191.48 88.36) (end 191.48 88.7) (width 0.1) (layer F.Cu) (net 2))
 (segment (start 194.8 91.16) (end 194.8 93.58) (width 0.1) (layer F.Cu) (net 2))
 (segment (start 194.36 90.72) (end 194.8 91.16) (width 0.1) (layer F.Cu) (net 2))
 (segment (start 193.5 90.72) (end 194.36 90.72) (width 0.1) (layer F.Cu) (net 2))
 (segment (start 191.48 88.7) (end 193.5 90.72) (width 0.1) (layer F.Cu) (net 2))
 (segment (start 191.48 88.36) (end 191.48 87.53) (width 0.1) (layer F.Cu) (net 2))
 (segment (start 191.575 87.435) (end 191.51 87.5) (width 0.1) (layer F.Cu) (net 2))
 (segment (start 191.575 87.435) (end 192.13 87.435) (width 0.1) (layer F.Cu) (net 2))
 (segment (start 191.48 87.53) (end 191.51 87.5) (width 0.1) (layer F.Cu) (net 2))
 (segment (start 189.458 91.43) (end 189.458 88.063) (width 0.1) (layer F.Cu) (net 2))
 (segment (start 189.458 88.063) (end 189.33 87.935) (width 0.1) (layer F.Cu) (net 2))
 (segment (start 193.778 84.67) (end 193.778 82.958) (width 0.254) (layer F.Cu) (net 2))
 (segment (start 188.952 84.67) (end 188.952 82.788) (width 0.254) (layer F.Cu) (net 2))
 (segment (start 189.458 91.43) (end 189.458 93.338) (width 0.254) (layer F.Cu) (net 2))
 (segment (start 189.7 93.58) (end 189.85 93.58) (width 0.254) (layer F.Cu) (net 2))
 (segment (start 189.458 93.338) (end 189.7 93.58) (width 0.254) (layer F.Cu) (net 2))
 (segment (start 189.85 93.58) (end 194.8 93.58) (width 0.254) (layer F.Cu) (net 2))
 (segment (start 204.93 85.2175) (end 203.43 83.7175) (width 0.254) (layer F.Cu) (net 2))
 (segment (start 194.8 93.58) (end 204.51 93.58) (width 0.254) (layer F.Cu) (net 2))
 (segment (start 204.51 93.58) (end 204.93 93.16) (width 0.254) (layer F.Cu) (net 2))
 (segment (start 204.93 93.16) (end 204.93 85.2175) (width 0.254) (layer F.Cu) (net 2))
 (segment (start 186.54 82.38) (end 189.36 82.38) (width 0.254) (layer F.Cu) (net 2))
 (segment (start 185.2025 83.7175) (end 186.54 82.38) (width 0.254) (layer F.Cu) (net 2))
 (segment (start 197.0125 82.38) (end 198.35 83.7175) (width 0.254) (layer F.Cu) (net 2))
 (segment (start 203.43 83.7175) (end 200.94 83.7175) (width 0.254) (layer F.Cu) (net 2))
 (segment (start 190.73 86.61) (end 190.73 82.53) (width 0.2) (layer F.Cu) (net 2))
 (segment (start 190.73 82.53) (end 190.58 82.38) (width 0.2) (layer F.Cu) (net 2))
 (segment (start 193.778 82.958) (end 193.2 82.38) (width 0.254) (layer F.Cu) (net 2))
 (segment (start 188.952 82.788) (end 189.36 82.38) (width 0.254) (layer F.Cu) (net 2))
 (segment (start 189.36 82.38) (end 190.58 82.38) (width 0.254) (layer F.Cu) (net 2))
 (segment (start 190.58 82.38) (end 193.2 82.38) (width 0.254) (layer F.Cu) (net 2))
 (segment (start 193.2 82.38) (end 197.0125 82.38) (width 0.254) (layer F.Cu) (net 2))
 (segment (start 193.988 92.01) (end 193.34 92.01) (width 0.1) (layer F.Cu) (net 5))
 (segment (start 190.48 89.05) (end 190.48 88.36) (width 0.1) (layer F.Cu) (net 5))
 (segment (start 190.27 89.26) (end 190.48 89.05) (width 0.1) (layer F.Cu) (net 5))
 (segment (start 190.27 92.37) (end 190.27 89.26) (width 0.1) (layer F.Cu) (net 5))
 (segment (start 190.51 92.61) (end 190.27 92.37) (width 0.1) (layer F.Cu) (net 5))
 (segment (start 192.74 92.61) (end 190.51 92.61) (width 0.1) (layer F.Cu) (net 5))
 (segment (start 193.34 92.01) (end 192.74 92.61) (width 0.1) (layer F.Cu) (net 5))
 (segment (start 190.982 91.43) (end 190.982 88.362) (width 0.1) (layer F.Cu) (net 6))
 (segment (start 190.982 88.362) (end 190.98 88.36) (width 0.1) (layer F.Cu) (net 6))
 (segment (start 186.412 89.75) (end 186.412 88.748) (width 0.1) (layer F.Cu) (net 4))
 (segment (start 187.725 87.435) (end 189.33 87.435) (width 0.1) (layer F.Cu) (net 4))
 (segment (start 186.412 88.748) (end 187.725 87.435) (width 0.1) (layer F.Cu) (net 4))
 (segment (start 189.33 87.435) (end 189.795 87.435) (width 0.1) (layer F.Cu) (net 4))
 (segment (start 189.795 87.435) (end 189.98 87.62) (width 0.1) (layer F.Cu) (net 4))
 (segment (start 189.98 88.36) (end 189.98 87.62) (width 0.1) (layer F.Cu) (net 4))
 (segment (start 189.98 87.62) (end 189.96 87.6) (width 0.1) (layer F.Cu) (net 4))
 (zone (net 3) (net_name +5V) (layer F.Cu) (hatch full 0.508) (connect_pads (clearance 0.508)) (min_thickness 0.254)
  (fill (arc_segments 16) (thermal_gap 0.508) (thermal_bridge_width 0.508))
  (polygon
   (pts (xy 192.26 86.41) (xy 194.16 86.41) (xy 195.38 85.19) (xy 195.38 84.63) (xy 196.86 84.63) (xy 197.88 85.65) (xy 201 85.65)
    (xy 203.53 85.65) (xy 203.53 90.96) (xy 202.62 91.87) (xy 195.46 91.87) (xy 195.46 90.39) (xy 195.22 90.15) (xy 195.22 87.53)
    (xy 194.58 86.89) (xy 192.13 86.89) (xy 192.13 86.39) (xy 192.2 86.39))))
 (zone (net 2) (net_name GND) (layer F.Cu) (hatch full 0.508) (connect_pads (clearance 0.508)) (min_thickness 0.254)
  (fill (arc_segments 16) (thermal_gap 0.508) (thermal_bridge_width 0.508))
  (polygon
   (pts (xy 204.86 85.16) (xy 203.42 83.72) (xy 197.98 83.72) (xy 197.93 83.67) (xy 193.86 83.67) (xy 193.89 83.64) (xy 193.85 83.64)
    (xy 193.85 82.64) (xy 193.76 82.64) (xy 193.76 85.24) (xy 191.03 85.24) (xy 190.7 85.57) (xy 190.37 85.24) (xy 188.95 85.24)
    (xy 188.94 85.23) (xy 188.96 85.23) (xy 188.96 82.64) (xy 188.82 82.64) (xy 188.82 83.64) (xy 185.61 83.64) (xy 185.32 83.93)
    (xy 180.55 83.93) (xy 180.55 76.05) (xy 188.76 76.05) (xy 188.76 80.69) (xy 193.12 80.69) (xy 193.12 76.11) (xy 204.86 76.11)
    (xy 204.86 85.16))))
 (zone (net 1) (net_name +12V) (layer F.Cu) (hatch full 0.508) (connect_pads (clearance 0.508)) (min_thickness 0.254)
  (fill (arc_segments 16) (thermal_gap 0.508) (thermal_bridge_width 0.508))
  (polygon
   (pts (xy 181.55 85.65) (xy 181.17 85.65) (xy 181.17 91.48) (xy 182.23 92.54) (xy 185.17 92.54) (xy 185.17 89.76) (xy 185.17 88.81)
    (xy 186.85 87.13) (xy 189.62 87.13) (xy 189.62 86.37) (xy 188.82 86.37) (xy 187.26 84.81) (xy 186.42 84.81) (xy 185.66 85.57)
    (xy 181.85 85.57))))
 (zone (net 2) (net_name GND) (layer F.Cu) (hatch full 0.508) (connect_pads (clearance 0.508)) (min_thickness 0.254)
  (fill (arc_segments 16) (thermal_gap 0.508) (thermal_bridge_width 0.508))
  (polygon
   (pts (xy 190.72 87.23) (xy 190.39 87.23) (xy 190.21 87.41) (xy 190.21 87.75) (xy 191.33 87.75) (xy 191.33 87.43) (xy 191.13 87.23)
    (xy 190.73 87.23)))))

